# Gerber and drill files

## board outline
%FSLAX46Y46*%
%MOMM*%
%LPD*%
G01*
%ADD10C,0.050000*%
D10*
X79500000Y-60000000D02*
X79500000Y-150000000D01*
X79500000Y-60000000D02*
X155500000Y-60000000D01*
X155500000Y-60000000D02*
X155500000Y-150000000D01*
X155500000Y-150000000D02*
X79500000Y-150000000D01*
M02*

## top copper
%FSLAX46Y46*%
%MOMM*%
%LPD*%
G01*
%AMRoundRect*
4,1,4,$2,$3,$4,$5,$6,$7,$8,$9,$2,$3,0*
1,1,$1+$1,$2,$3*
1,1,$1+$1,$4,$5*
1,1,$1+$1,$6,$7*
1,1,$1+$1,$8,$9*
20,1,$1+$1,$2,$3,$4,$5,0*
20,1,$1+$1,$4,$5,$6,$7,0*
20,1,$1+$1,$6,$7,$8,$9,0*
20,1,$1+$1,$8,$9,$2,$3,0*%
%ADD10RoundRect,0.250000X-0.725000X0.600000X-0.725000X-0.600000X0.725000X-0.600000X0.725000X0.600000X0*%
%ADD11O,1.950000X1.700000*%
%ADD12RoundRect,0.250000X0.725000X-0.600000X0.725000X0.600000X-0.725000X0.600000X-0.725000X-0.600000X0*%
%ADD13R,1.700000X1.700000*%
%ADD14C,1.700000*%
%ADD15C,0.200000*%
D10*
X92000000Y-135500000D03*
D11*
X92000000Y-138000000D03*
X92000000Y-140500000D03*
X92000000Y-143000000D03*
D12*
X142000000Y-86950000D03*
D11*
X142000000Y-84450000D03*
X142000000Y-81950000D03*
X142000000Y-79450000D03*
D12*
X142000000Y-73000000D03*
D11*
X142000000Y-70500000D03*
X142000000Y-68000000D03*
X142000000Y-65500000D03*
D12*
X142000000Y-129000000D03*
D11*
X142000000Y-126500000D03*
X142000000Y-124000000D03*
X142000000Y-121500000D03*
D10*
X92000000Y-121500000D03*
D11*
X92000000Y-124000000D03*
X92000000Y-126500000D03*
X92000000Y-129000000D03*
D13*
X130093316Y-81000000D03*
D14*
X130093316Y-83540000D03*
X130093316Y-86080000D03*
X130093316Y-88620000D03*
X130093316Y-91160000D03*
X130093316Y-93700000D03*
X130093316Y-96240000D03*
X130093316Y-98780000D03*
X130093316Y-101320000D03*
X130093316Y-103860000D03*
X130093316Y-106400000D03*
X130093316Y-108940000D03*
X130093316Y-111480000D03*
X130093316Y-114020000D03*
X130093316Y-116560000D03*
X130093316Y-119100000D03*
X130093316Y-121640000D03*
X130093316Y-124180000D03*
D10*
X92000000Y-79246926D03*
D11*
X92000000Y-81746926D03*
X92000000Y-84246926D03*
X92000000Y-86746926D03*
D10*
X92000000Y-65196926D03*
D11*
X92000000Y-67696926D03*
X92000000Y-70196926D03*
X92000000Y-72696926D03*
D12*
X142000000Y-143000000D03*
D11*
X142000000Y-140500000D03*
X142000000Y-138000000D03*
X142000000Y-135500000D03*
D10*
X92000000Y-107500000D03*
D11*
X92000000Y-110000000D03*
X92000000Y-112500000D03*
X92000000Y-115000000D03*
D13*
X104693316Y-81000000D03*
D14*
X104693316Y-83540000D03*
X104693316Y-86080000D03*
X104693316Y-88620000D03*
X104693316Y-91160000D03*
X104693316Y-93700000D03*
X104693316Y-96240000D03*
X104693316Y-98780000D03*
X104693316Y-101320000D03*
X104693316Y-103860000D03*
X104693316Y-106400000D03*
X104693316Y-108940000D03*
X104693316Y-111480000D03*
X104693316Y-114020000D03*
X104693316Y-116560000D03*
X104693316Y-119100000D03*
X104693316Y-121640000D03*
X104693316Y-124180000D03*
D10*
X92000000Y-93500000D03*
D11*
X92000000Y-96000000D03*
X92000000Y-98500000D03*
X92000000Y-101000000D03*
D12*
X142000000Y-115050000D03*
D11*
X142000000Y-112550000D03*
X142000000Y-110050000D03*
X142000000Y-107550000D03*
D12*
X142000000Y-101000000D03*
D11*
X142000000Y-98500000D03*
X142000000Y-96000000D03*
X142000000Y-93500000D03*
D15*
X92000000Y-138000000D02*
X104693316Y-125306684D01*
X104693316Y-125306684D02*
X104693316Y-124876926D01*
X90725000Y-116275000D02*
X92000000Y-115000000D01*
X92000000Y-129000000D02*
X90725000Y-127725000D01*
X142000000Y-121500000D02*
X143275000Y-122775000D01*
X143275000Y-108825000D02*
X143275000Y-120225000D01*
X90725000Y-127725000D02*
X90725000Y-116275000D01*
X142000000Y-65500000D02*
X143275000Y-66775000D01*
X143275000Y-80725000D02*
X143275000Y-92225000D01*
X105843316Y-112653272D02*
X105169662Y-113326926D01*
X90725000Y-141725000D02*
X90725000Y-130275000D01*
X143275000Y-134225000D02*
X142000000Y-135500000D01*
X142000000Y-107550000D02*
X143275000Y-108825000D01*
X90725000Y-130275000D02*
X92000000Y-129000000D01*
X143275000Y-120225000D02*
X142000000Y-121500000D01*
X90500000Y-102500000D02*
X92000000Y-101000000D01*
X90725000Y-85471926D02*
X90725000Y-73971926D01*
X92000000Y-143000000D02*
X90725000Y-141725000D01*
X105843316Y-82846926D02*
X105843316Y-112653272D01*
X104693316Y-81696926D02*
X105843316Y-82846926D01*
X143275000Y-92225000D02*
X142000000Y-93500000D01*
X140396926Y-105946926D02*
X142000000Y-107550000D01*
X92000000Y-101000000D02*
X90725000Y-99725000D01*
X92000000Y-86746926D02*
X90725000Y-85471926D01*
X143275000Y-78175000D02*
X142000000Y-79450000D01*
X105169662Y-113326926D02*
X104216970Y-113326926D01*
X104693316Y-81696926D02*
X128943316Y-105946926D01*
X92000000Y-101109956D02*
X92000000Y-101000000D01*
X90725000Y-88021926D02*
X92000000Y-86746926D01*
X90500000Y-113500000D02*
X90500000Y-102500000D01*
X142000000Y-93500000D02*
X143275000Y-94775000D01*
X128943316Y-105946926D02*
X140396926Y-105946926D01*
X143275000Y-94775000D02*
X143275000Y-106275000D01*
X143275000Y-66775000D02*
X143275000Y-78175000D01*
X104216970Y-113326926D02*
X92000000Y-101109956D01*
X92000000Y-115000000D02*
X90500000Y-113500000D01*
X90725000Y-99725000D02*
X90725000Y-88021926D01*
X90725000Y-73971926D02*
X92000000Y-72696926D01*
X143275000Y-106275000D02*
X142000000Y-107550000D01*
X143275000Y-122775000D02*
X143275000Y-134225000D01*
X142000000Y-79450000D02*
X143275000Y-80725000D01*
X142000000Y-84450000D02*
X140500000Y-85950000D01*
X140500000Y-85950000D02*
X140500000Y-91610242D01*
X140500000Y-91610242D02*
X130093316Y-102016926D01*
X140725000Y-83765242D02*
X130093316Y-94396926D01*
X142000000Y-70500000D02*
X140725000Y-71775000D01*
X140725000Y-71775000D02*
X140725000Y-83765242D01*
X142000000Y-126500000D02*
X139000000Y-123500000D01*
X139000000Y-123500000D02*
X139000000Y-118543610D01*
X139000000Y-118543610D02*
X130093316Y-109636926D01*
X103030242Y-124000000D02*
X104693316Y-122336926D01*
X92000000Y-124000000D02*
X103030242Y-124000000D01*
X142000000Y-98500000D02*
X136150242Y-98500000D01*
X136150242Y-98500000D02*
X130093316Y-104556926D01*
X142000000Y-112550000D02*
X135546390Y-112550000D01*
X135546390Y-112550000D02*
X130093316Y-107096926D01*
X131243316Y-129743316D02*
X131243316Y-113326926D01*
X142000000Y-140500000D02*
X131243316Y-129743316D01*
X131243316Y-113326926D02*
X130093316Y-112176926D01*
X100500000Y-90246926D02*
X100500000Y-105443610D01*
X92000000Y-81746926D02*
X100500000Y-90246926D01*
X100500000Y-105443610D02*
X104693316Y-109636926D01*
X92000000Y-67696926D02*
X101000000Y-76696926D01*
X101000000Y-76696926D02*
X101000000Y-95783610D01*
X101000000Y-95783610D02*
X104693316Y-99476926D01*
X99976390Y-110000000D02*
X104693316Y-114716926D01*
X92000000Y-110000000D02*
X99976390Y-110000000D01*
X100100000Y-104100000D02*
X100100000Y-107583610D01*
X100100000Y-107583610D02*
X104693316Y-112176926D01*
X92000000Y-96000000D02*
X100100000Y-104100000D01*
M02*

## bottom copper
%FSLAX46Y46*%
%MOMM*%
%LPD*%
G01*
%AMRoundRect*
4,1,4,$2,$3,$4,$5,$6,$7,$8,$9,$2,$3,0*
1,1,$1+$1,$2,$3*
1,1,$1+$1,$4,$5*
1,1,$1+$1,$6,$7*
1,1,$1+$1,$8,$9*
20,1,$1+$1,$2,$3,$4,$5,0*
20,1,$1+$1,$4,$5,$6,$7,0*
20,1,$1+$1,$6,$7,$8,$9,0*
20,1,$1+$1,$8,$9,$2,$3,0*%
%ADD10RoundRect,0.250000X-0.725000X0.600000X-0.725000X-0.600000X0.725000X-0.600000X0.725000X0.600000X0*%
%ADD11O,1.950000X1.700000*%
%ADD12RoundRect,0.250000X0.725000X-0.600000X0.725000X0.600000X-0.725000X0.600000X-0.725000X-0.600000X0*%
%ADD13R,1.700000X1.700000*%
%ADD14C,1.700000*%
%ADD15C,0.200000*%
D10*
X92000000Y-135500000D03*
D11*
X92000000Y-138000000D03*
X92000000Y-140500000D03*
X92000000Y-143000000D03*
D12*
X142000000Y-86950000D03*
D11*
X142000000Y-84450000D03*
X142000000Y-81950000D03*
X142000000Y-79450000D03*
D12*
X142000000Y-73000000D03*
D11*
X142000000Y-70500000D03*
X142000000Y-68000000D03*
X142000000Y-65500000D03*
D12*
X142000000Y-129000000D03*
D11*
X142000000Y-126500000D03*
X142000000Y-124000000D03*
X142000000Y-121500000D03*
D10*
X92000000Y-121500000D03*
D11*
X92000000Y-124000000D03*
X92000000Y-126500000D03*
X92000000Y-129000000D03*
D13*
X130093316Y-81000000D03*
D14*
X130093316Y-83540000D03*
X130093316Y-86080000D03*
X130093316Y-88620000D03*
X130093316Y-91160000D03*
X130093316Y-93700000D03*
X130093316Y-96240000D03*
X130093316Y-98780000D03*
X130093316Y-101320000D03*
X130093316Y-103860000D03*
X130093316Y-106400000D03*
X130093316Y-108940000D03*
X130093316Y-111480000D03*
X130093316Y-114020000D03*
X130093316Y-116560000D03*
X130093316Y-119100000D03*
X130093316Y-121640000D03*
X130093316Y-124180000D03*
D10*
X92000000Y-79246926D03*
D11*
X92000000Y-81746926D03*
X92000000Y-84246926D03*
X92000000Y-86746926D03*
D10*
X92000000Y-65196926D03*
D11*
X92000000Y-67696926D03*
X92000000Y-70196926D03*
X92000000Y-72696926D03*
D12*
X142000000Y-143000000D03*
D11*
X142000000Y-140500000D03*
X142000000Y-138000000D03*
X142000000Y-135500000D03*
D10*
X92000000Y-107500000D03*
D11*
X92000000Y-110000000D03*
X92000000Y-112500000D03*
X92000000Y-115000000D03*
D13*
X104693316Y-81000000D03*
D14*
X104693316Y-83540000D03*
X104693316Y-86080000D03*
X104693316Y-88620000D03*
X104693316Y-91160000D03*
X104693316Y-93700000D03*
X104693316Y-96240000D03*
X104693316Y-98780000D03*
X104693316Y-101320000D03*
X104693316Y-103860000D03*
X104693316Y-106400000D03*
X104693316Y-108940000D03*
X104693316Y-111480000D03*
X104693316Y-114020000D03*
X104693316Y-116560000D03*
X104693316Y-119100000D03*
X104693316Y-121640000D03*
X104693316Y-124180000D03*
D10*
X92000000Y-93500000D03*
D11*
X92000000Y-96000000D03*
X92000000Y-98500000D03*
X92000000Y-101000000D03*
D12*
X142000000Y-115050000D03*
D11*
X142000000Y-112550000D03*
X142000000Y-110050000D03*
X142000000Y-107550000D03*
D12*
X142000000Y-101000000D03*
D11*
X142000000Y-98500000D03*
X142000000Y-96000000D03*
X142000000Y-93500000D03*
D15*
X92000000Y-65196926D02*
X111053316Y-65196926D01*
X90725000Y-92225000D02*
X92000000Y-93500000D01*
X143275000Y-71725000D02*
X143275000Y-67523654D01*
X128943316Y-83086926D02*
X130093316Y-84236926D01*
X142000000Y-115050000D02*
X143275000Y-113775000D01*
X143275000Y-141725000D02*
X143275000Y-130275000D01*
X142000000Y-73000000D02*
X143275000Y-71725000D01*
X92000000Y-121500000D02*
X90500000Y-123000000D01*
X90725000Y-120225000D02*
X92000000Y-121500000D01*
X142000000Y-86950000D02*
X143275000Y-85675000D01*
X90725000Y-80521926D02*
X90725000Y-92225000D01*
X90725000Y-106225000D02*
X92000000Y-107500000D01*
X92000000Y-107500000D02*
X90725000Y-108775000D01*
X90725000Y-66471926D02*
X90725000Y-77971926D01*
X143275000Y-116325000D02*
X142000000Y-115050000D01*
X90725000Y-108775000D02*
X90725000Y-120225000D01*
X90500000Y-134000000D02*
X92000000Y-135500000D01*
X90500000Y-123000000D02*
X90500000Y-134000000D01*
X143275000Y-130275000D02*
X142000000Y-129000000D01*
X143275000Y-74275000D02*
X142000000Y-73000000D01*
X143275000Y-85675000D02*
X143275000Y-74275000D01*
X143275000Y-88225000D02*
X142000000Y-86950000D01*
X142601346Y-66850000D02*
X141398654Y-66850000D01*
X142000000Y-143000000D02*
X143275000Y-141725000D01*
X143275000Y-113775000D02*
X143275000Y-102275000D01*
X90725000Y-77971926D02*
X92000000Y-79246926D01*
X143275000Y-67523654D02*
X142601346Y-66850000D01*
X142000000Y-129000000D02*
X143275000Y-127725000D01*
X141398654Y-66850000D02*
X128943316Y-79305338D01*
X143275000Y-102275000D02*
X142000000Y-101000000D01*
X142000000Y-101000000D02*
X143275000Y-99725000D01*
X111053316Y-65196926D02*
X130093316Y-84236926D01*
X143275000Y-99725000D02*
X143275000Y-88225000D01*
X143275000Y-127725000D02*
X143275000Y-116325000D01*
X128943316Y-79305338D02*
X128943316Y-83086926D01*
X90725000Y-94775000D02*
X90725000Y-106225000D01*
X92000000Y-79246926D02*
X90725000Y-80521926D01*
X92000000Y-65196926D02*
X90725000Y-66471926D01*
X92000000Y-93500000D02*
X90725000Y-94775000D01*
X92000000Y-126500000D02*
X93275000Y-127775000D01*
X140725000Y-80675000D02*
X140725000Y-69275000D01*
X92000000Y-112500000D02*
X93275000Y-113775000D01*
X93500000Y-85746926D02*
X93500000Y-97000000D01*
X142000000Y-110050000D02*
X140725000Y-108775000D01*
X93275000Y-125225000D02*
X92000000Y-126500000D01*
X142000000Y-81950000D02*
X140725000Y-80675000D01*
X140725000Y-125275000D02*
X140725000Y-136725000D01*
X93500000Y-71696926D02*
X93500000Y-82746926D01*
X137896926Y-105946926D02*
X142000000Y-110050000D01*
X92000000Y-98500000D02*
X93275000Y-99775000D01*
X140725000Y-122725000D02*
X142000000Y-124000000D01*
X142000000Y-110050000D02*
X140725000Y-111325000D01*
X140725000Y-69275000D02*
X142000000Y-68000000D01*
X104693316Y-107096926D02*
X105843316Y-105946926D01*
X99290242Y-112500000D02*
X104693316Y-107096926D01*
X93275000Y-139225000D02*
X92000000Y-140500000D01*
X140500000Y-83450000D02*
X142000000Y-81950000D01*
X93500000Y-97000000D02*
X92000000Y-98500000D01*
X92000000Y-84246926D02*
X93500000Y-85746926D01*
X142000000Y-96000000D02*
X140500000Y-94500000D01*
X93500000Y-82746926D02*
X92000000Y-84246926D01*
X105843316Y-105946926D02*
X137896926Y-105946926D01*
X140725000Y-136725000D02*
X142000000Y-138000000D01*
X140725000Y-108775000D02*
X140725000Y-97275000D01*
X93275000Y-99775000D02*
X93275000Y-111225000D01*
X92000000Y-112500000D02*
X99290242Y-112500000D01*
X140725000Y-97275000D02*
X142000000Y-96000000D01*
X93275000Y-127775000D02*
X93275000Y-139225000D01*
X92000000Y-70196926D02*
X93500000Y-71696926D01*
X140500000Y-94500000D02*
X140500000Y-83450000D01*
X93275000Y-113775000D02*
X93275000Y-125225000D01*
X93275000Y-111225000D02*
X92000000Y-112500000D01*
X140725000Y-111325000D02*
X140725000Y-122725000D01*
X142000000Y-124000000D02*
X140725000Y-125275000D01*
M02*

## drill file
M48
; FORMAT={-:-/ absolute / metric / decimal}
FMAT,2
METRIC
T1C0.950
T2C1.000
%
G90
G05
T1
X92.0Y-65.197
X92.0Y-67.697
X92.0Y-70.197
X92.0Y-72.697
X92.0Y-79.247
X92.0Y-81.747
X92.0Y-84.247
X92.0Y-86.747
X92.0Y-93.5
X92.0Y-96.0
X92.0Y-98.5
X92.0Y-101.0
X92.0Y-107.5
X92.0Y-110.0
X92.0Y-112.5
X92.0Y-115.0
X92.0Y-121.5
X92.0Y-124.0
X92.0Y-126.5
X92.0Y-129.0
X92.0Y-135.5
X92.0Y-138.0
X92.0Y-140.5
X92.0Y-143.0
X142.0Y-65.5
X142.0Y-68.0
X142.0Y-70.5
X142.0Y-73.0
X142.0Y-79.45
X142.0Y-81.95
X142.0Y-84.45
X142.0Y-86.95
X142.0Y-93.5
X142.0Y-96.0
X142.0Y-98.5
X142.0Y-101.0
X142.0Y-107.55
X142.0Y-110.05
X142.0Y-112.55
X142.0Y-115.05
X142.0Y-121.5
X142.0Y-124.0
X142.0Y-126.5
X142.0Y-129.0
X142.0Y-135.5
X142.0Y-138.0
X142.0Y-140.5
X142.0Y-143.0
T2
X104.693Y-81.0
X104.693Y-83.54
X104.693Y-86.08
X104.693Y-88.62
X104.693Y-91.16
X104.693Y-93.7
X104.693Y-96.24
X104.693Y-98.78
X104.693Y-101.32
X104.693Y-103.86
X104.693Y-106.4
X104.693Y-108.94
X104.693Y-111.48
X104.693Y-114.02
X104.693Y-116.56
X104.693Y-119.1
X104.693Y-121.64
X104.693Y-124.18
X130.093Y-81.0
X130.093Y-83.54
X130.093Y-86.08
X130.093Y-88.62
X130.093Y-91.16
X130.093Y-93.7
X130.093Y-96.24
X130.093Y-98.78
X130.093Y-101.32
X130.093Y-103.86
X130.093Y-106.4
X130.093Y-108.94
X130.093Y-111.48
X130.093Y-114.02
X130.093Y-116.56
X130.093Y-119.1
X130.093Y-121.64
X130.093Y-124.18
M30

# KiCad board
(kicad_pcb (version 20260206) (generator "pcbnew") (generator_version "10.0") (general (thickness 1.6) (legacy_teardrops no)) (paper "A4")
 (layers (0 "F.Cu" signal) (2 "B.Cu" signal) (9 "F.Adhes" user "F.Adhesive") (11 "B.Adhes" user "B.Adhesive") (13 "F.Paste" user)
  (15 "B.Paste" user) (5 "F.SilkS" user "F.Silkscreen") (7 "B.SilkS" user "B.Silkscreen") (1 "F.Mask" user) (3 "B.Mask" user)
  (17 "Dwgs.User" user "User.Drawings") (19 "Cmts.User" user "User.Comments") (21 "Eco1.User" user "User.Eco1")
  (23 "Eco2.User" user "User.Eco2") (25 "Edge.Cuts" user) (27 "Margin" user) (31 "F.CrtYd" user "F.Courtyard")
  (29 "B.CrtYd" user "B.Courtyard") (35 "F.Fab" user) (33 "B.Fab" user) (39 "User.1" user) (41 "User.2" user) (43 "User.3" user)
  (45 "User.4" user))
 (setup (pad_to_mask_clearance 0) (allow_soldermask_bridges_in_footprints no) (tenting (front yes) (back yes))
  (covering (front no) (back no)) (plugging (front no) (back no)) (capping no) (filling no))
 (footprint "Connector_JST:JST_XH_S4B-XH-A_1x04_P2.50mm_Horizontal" (layer "F.Cu") (at 92 135.5 -90)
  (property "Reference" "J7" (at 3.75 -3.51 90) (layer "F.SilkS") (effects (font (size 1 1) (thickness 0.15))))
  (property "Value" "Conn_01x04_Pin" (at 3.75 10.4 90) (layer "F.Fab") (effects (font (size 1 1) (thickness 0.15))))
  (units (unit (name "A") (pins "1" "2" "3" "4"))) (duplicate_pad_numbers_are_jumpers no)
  (pad "1" thru_hole roundrect (at 0 0 270) (size 1.7 1.95) (drill 0.95) (layers "*.Cu" "*.Mask") (remove_unused_layers no)
   (roundrect_rratio 0.147059) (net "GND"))
  (pad "2" thru_hole oval (at 2.5 0 270) (size 1.7 1.95) (drill 0.95) (layers "*.Cu" "*.Mask") (remove_unused_layers no) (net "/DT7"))
  (pad "3" thru_hole oval (at 5 0 270) (size 1.7 1.95) (drill 0.95) (layers "*.Cu" "*.Mask") (remove_unused_layers no) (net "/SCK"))
  (pad "4" thru_hole oval (at 7.5 0 270) (size 1.7 1.95) (drill 0.95) (layers "*.Cu" "*.Mask") (remove_unused_layers no) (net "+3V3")))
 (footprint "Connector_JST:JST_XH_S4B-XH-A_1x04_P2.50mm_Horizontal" (layer "F.Cu") (at 142 86.95 90)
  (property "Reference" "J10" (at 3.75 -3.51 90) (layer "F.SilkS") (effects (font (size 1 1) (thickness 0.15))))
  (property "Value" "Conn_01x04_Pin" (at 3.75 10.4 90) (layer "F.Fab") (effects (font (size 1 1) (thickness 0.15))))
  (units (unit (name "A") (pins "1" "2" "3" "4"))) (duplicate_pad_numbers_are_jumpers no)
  (pad "1" thru_hole roundrect (at 0 0 90) (size 1.7 1.95) (drill 0.95) (layers "*.Cu" "*.Mask") (remove_unused_layers no)
   (roundrect_rratio 0.147059) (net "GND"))
  (pad "2" thru_hole oval (at 2.5 0 90) (size 1.7 1.95) (drill 0.95) (layers "*.Cu" "*.Mask") (remove_unused_layers no) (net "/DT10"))
  (pad "3" thru_hole oval (at 5 0 90) (size 1.7 1.95) (drill 0.95) (layers "*.Cu" "*.Mask") (remove_unused_layers no) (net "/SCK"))
  (pad "4" thru_hole oval (at 7.5 0 90) (size 1.7 1.95) (drill 0.95) (layers "*.Cu" "*.Mask") (remove_unused_layers no) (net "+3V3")))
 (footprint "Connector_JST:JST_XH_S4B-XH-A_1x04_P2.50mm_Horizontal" (layer "F.Cu") (at 142 73 90)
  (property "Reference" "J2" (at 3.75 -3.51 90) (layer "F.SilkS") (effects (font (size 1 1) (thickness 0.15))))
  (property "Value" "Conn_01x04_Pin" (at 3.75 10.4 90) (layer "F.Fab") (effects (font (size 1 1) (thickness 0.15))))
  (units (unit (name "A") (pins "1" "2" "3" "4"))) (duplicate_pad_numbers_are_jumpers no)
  (pad "1" thru_hole roundrect (at 0 0 90) (size 1.7 1.95) (drill 0.95) (layers "*.Cu" "*.Mask") (remove_unused_layers no)
   (roundrect_rratio 0.147059) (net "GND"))
  (pad "2" thru_hole oval (at 2.5 0 90) (size 1.7 1.95) (drill 0.95) (layers "*.Cu" "*.Mask") (remove_unused_layers no) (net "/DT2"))
  (pad "3" thru_hole oval (at 5 0 90) (size 1.7 1.95) (drill 0.95) (layers "*.Cu" "*.Mask") (remove_unused_layers no) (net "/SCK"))
  (pad "4" thru_hole oval (at 7.5 0 90) (size 1.7 1.95) (drill 0.95) (layers "*.Cu" "*.Mask") (remove_unused_layers no) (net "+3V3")))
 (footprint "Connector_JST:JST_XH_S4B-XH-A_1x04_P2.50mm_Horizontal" (layer "F.Cu") (at 142 129 90)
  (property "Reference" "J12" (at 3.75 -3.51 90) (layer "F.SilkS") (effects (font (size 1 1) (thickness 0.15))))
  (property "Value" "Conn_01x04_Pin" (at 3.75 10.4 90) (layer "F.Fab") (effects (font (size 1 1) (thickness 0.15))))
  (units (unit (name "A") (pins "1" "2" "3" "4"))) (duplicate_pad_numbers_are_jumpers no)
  (pad "1" thru_hole roundrect (at 0 0 90) (size 1.7 1.95) (drill 0.95) (layers "*.Cu" "*.Mask") (remove_unused_layers no)
   (roundrect_rratio 0.147059) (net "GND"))
  (pad "2" thru_hole oval (at 2.5 0 90) (size 1.7 1.95) (drill 0.95) (layers "*.Cu" "*.Mask") (remove_unused_layers no) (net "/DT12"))
  (pad "3" thru_hole oval (at 5 0 90) (size 1.7 1.95) (drill 0.95) (layers "*.Cu" "*.Mask") (remove_unused_layers no) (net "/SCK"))
  (pad "4" thru_hole oval (at 7.5 0 90) (size 1.7 1.95) (drill 0.95) (layers "*.Cu" "*.Mask") (remove_unused_layers no) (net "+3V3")))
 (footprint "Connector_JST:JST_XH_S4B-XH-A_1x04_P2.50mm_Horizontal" (layer "F.Cu") (at 92 121.5 -90)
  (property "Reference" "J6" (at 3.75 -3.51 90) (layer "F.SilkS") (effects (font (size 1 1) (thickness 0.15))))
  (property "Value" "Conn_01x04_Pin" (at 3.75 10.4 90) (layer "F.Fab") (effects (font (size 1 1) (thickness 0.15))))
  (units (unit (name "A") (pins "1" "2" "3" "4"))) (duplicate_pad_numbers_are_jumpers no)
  (pad "1" thru_hole roundrect (at 0 0 270) (size 1.7 1.95) (drill 0.95) (layers "*.Cu" "*.Mask") (remove_unused_layers no)
   (roundrect_rratio 0.147059) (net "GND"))
  (pad "2" thru_hole oval (at 2.5 0 270) (size 1.7 1.95) (drill 0.95) (layers "*.Cu" "*.Mask") (remove_unused_layers no) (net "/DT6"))
  (pad "3" thru_hole oval (at 5 0 270) (size 1.7 1.95) (drill 0.95) (layers "*.Cu" "*.Mask") (remove_unused_layers no) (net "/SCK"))
  (pad "4" thru_hole oval (at 7.5 0 270) (size 1.7 1.95) (drill 0.95) (layers "*.Cu" "*.Mask") (remove_unused_layers no) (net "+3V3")))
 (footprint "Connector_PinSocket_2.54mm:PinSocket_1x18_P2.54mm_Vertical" (layer "F.Cu") (at 130.093316 81)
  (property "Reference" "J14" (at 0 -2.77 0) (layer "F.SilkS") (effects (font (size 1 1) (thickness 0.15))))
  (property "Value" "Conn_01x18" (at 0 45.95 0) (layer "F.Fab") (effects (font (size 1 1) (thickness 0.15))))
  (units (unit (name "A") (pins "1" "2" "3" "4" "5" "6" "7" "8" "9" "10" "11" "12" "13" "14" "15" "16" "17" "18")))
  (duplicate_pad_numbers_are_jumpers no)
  (pad "1" thru_hole rect (at 0 0) (size 1.7 1.7) (drill 1) (layers "*.Cu" "*.Mask") (remove_unused_layers no)
   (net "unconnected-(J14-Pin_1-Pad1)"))
  (pad "2" thru_hole circle (at 0 2.54) (size 1.7 1.7) (drill 1) (layers "*.Cu" "*.Mask") (remove_unused_layers no) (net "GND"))
  (pad "3" thru_hole circle (at 0 5.08) (size 1.7 1.7) (drill 1) (layers "*.Cu" "*.Mask") (remove_unused_layers no)
   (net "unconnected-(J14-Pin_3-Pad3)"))
  (pad "4" thru_hole circle (at 0 7.62) (size 1.7 1.7) (drill 1) (layers "*.Cu" "*.Mask") (remove_unused_layers no)
   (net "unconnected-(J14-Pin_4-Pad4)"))
  (pad "5" thru_hole circle (at 0 10.16) (size 1.7 1.7) (drill 1) (layers "*.Cu" "*.Mask") (remove_unused_layers no)
   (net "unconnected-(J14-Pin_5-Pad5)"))
  (pad "6" thru_hole circle (at 0 12.7) (size 1.7 1.7) (drill 1) (layers "*.Cu" "*.Mask") (remove_unused_layers no) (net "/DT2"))
  (pad "7" thru_hole circle (at 0 15.24) (size 1.7 1.7) (drill 1) (layers "*.Cu" "*.Mask") (remove_unused_layers no)
   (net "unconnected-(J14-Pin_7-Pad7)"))
  (pad "8" thru_hole circle (at 0 17.78) (size 1.7 1.7) (drill 1) (layers "*.Cu" "*.Mask") (remove_unused_layers no)
   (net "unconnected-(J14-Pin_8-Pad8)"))
  (pad "9" thru_hole circle (at 0 20.32) (size 1.7 1.7) (drill 1) (layers "*.Cu" "*.Mask") (remove_unused_layers no) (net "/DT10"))
  (pad "10" thru_hole circle (at 0 22.86) (size 1.7 1.7) (drill 1) (layers "*.Cu" "*.Mask") (remove_unused_layers no) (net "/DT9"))
  (pad "11" thru_hole circle (at 0 25.4) (size 1.7 1.7) (drill 1) (layers "*.Cu" "*.Mask") (remove_unused_layers no) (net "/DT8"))
  (pad "12" thru_hole circle (at 0 27.94) (size 1.7 1.7) (drill 1) (layers "*.Cu" "*.Mask") (remove_unused_layers no) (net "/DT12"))
  (pad "13" thru_hole circle (at 0 30.48) (size 1.7 1.7) (drill 1) (layers "*.Cu" "*.Mask") (remove_unused_layers no) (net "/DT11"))
  (pad "14" thru_hole circle (at 0 33.02) (size 1.7 1.7) (drill 1) (layers "*.Cu" "*.Mask") (remove_unused_layers no)
   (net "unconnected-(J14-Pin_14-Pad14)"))
  (pad "15" thru_hole circle (at 0 35.56) (size 1.7 1.7) (drill 1) (layers "*.Cu" "*.Mask") (remove_unused_layers no)
   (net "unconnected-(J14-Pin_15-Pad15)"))
  (pad "16" thru_hole circle (at 0 38.1) (size 1.7 1.7) (drill 1) (layers "*.Cu" "*.Mask") (remove_unused_layers no)
   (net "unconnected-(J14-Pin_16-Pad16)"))
  (pad "17" thru_hole circle (at 0 40.64) (size 1.7 1.7) (drill 1) (layers "*.Cu" "*.Mask") (remove_unused_layers no)
   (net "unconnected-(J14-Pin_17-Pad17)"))
  (pad "18" thru_hole circle (at 0 43.18) (size 1.7 1.7) (drill 1) (layers "*.Cu" "*.Mask") (remove_unused_layers no)
   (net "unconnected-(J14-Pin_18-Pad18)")))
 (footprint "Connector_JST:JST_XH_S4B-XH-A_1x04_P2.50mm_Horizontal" (layer "F.Cu") (at 92 79.246926 -90)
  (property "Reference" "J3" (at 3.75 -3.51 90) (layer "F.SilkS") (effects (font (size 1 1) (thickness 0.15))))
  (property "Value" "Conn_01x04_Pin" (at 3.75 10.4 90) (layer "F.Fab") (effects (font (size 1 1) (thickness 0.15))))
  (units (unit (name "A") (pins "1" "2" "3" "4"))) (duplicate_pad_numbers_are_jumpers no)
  (pad "1" thru_hole roundrect (at 0 0 270) (size 1.7 1.95) (drill 0.95) (layers "*.Cu" "*.Mask") (remove_unused_layers no)
   (roundrect_rratio 0.147059) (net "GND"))
  (pad "2" thru_hole oval (at 2.5 0 270) (size 1.7 1.95) (drill 0.95) (layers "*.Cu" "*.Mask") (remove_unused_layers no) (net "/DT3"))
  (pad "3" thru_hole oval (at 5 0 270) (size 1.7 1.95) (drill 0.95) (layers "*.Cu" "*.Mask") (remove_unused_layers no) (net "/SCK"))
  (pad "4" thru_hole oval (at 7.5 0 270) (size 1.7 1.95) (drill 0.95) (layers "*.Cu" "*.Mask") (remove_unused_layers no) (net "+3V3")))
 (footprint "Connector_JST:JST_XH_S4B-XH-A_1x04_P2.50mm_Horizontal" (layer "F.Cu") (at 92 65.196926 -90)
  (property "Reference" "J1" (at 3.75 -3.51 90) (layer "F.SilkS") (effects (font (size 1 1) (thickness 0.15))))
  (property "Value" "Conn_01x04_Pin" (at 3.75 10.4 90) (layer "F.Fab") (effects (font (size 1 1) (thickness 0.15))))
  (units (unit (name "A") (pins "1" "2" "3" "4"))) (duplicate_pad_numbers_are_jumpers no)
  (pad "1" thru_hole roundrect (at 0 0 270) (size 1.7 1.95) (drill 0.95) (layers "*.Cu" "*.Mask") (remove_unused_layers no)
   (roundrect_rratio 0.147059) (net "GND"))
  (pad "2" thru_hole oval (at 2.5 0 270) (size 1.7 1.95) (drill 0.95) (layers "*.Cu" "*.Mask") (remove_unused_layers no) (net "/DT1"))
  (pad "3" thru_hole oval (at 5 0 270) (size 1.7 1.95) (drill 0.95) (layers "*.Cu" "*.Mask") (remove_unused_layers no) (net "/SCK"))
  (pad "4" thru_hole oval (at 7.5 0 270) (size 1.7 1.95) (drill 0.95) (layers "*.Cu" "*.Mask") (remove_unused_layers no) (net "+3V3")))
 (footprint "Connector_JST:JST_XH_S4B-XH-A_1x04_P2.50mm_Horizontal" (layer "F.Cu") (at 142 143 90)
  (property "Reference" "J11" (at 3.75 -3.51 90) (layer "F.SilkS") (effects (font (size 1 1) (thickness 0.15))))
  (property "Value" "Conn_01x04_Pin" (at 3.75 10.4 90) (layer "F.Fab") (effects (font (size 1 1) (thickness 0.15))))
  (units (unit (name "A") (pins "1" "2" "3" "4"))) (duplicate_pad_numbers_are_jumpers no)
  (pad "1" thru_hole roundrect (at 0 0 90) (size 1.7 1.95) (drill 0.95) (layers "*.Cu" "*.Mask") (remove_unused_layers no)
   (roundrect_rratio 0.147059) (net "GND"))
  (pad "2" thru_hole oval (at 2.5 0 90) (size 1.7 1.95) (drill 0.95) (layers "*.Cu" "*.Mask") (remove_unused_layers no) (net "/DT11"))
  (pad "3" thru_hole oval (at 5 0 90) (size 1.7 1.95) (drill 0.95) (layers "*.Cu" "*.Mask") (remove_unused_layers no) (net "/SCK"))
  (pad "4" thru_hole oval (at 7.5 0 90) (size 1.7 1.95) (drill 0.95) (layers "*.Cu" "*.Mask") (remove_unused_layers no) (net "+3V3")))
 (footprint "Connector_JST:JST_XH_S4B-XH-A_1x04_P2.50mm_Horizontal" (layer "F.Cu") (at 92 107.5 -90)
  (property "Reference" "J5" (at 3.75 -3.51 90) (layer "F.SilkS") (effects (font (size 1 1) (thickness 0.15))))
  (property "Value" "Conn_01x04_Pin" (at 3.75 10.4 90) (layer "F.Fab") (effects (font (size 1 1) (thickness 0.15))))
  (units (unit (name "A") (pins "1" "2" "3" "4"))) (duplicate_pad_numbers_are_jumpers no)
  (pad "1" thru_hole roundrect (at 0 0 270) (size 1.7 1.95) (drill 0.95) (layers "*.Cu" "*.Mask") (remove_unused_layers no)
   (roundrect_rratio 0.147059) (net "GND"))
  (pad "2" thru_hole oval (at 2.5 0 270) (size 1.7 1.95) (drill 0.95) (layers "*.Cu" "*.Mask") (remove_unused_layers no) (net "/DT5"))
  (pad "3" thru_hole oval (at 5 0 270) (size 1.7 1.95) (drill 0.95) (layers "*.Cu" "*.Mask") (remove_unused_layers no) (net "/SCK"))
  (pad "4" thru_hole oval (at 7.5 0 270) (size 1.7 1.95) (drill 0.95) (layers "*.Cu" "*.Mask") (remove_unused_layers no) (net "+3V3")))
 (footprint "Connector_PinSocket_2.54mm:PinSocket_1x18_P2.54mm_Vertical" (layer "F.Cu") (at 104.693316 81)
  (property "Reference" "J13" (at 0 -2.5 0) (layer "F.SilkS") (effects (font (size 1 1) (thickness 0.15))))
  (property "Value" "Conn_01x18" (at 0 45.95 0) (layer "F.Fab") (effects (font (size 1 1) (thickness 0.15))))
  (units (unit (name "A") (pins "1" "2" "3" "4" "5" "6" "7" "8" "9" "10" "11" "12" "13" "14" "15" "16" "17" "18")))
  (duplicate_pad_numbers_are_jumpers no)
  (pad "1" thru_hole rect (at 0 0) (size 1.7 1.7) (drill 1) (layers "*.Cu" "*.Mask") (remove_unused_layers no) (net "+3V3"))
  (pad "2" thru_hole circle (at 0 2.54) (size 1.7 1.7) (drill 1) (layers "*.Cu" "*.Mask") (remove_unused_layers no)
   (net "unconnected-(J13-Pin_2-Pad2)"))
  (pad "3" thru_hole circle (at 0 5.08) (size 1.7 1.7) (drill 1) (layers "*.Cu" "*.Mask") (remove_unused_layers no)
   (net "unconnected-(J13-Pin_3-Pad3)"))
  (pad "4" thru_hole circle (at 0 7.62) (size 1.7 1.7) (drill 1) (layers "*.Cu" "*.Mask") (remove_unused_layers no)
   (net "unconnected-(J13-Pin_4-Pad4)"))
  (pad "5" thru_hole circle (at 0 10.16) (size 1.7 1.7) (drill 1) (layers "*.Cu" "*.Mask") (remove_unused_layers no)
   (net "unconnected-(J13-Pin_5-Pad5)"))
  (pad "6" thru_hole circle (at 0 12.7) (size 1.7 1.7) (drill 1) (layers "*.Cu" "*.Mask") (remove_unused_layers no)
   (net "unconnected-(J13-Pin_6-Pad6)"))
  (pad "7" thru_hole circle (at 0 15.24) (size 1.7 1.7) (drill 1) (layers "*.Cu" "*.Mask") (remove_unused_layers no)
   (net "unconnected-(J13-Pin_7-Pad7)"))
  (pad "8" thru_hole circle (at 0 17.78) (size 1.7 1.7) (drill 1) (layers "*.Cu" "*.Mask") (remove_unused_layers no) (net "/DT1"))
  (pad "9" thru_hole circle (at 0 20.32) (size 1.7 1.7) (drill 1) (layers "*.Cu" "*.Mask") (remove_unused_layers no)
   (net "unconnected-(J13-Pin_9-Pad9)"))
  (pad "10" thru_hole circle (at 0 22.86) (size 1.7 1.7) (drill 1) (layers "*.Cu" "*.Mask") (remove_unused_layers no)
   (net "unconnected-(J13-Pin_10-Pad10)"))
  (pad "11" thru_hole circle (at 0 25.4) (size 1.7 1.7) (drill 1) (layers "*.Cu" "*.Mask") (remove_unused_layers no) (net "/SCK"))
  (pad "12" thru_hole circle (at 0 27.94) (size 1.7 1.7) (drill 1) (layers "*.Cu" "*.Mask") (remove_unused_layers no) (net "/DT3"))
  (pad "13" thru_hole circle (at 0 30.48) (size 1.7 1.7) (drill 1) (layers "*.Cu" "*.Mask") (remove_unused_layers no) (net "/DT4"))
  (pad "14" thru_hole circle (at 0 33.02) (size 1.7 1.7) (drill 1) (layers "*.Cu" "*.Mask") (remove_unused_layers no) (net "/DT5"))
  (pad "15" thru_hole circle (at 0 35.56) (size 1.7 1.7) (drill 1) (layers "*.Cu" "*.Mask") (remove_unused_layers no)
   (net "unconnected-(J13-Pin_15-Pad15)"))
  (pad "16" thru_hole circle (at 0 38.1) (size 1.7 1.7) (drill 1) (layers "*.Cu" "*.Mask") (remove_unused_layers no)
   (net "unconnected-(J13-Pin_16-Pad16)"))
  (pad "17" thru_hole circle (at 0 40.64) (size 1.7 1.7) (drill 1) (layers "*.Cu" "*.Mask") (remove_unused_layers no) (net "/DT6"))
  (pad "18" thru_hole circle (at 0 43.18) (size 1.7 1.7) (drill 1) (layers "*.Cu" "*.Mask") (remove_unused_layers no) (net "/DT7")))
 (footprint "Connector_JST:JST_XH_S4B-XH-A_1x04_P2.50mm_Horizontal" (layer "F.Cu") (at 92 93.5 -90)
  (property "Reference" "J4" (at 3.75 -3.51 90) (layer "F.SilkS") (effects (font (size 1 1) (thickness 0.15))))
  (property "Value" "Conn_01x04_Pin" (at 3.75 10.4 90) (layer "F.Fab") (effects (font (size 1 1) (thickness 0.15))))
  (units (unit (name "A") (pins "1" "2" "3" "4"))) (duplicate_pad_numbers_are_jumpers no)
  (pad "1" thru_hole roundrect (at 0 0 270) (size 1.7 1.95) (drill 0.95) (layers "*.Cu" "*.Mask") (remove_unused_layers no)
   (roundrect_rratio 0.147059) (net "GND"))
  (pad "2" thru_hole oval (at 2.5 0 270) (size 1.7 1.95) (drill 0.95) (layers "*.Cu" "*.Mask") (remove_unused_layers no) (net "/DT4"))
  (pad "3" thru_hole oval (at 5 0 270) (size 1.7 1.95) (drill 0.95) (layers "*.Cu" "*.Mask") (remove_unused_layers no) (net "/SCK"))
  (pad "4" thru_hole oval (at 7.5 0 270) (size 1.7 1.95) (drill 0.95) (layers "*.Cu" "*.Mask") (remove_unused_layers no) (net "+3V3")))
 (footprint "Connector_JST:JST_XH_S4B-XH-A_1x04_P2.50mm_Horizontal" (layer "F.Cu") (at 142 115.05 90)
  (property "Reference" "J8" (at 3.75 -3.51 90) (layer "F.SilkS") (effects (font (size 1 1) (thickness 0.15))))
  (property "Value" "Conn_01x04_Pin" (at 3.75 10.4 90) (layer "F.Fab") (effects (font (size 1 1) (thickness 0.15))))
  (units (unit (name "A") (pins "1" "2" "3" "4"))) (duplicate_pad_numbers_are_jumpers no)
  (pad "1" thru_hole roundrect (at 0 0 90) (size 1.7 1.95) (drill 0.95) (layers "*.Cu" "*.Mask") (remove_unused_layers no)
   (roundrect_rratio 0.147059) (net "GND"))
  (pad "2" thru_hole oval (at 2.5 0 90) (size 1.7 1.95) (drill 0.95) (layers "*.Cu" "*.Mask") (remove_unused_layers no) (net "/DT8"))
  (pad "3" thru_hole oval (at 5 0 90) (size 1.7 1.95) (drill 0.95) (layers "*.Cu" "*.Mask") (remove_unused_layers no) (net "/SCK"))
  (pad "4" thru_hole oval (at 7.5 0 90) (size 1.7 1.95) (drill 0.95) (layers "*.Cu" "*.Mask") (remove_unused_layers no) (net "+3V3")))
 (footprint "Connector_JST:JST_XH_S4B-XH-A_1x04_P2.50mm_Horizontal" (layer "F.Cu") (at 142 101 90)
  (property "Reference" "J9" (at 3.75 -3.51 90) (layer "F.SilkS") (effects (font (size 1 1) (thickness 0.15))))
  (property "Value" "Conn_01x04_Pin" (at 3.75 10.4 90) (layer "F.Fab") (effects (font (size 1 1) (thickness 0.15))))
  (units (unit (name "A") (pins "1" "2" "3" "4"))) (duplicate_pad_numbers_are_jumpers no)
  (pad "1" thru_hole roundrect (at 0 0 90) (size 1.7 1.95) (drill 0.95) (layers "*.Cu" "*.Mask") (remove_unused_layers no)
   (roundrect_rratio 0.147059) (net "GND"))
  (pad "2" thru_hole oval (at 2.5 0 90) (size 1.7 1.95) (drill 0.95) (layers "*.Cu" "*.Mask") (remove_unused_layers no) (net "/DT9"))
  (pad "3" thru_hole oval (at 5 0 90) (size 1.7 1.95) (drill 0.95) (layers "*.Cu" "*.Mask") (remove_unused_layers no) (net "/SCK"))
  (pad "4" thru_hole oval (at 7.5 0 90) (size 1.7 1.95) (drill 0.95) (layers "*.Cu" "*.Mask") (remove_unused_layers no) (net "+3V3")))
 (gr_line (start 79.5 60) (end 79.5 150) (stroke (width 0.05) (type default)) (layer "Edge.Cuts"))
 (gr_line (start 79.5 60) (end 155.5 60) (stroke (width 0.05) (type default)) (layer "Edge.Cuts"))
 (gr_line (start 155.5 60) (end 155.5 150) (stroke (width 0.05) (type default)) (layer "Edge.Cuts"))
 (gr_line (start 155.5 150) (end 79.5 150) (stroke (width 0.05) (type default)) (layer "Edge.Cuts"))
 (segment (start 92 65.196926) (end 111.053316 65.196926) (width 0.2) (layer "B.Cu") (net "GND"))
 (segment (start 90.725 92.225) (end 92 93.5) (width 0.2) (layer "B.Cu") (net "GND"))
 (segment (start 143.275 71.725) (end 143.275 67.523654) (width 0.2) (layer "B.Cu") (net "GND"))
 (segment (start 128.943316 83.086926) (end 130.093316 84.236926) (width 0.2) (layer "B.Cu") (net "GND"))
 (segment (start 142 115.05) (end 143.275 113.775) (width 0.2) (layer "B.Cu") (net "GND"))
 (segment (start 143.275 141.725) (end 143.275 130.275) (width 0.2) (layer "B.Cu") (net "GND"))
 (segment (start 142 73) (end 143.275 71.725) (width 0.2) (layer "B.Cu") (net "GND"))
 (segment (start 92 121.5) (end 90.5 123) (width 0.2) (layer "B.Cu") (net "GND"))
 (segment (start 90.725 120.225) (end 92 121.5) (width 0.2) (layer "B.Cu") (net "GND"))
 (segment (start 142 86.95) (end 143.275 85.675) (width 0.2) (layer "B.Cu") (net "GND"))
 (segment (start 90.725 80.521926) (end 90.725 92.225) (width 0.2) (layer "B.Cu") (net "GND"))
 (segment (start 90.725 106.225) (end 92 107.5) (width 0.2) (layer "B.Cu") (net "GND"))
 (segment (start 92 107.5) (end 90.725 108.775) (width 0.2) (layer "B.Cu") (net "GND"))
 (segment (start 90.725 66.471926) (end 90.725 77.971926) (width 0.2) (layer "B.Cu") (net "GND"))
 (segment (start 143.275 116.325) (end 142 115.05) (width 0.2) (layer "B.Cu") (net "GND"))
 (segment (start 90.725 108.775) (end 90.725 120.225) (width 0.2) (layer "B.Cu") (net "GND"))
 (segment (start 90.5 134) (end 92 135.5) (width 0.2) (layer "B.Cu") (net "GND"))
 (segment (start 90.5 123) (end 90.5 134) (width 0.2) (layer "B.Cu") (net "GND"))
 (segment (start 143.275 130.275) (end 142 129) (width 0.2) (layer "B.Cu") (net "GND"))
 (segment (start 143.275 74.275) (end 142 73) (width 0.2) (layer "B.Cu") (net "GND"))
 (segment (start 143.275 85.675) (end 143.275 74.275) (width 0.2) (layer "B.Cu") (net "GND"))
 (segment (start 143.275 88.225) (end 142 86.95) (width 0.2) (layer "B.Cu") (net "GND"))
 (segment (start 142.601346 66.85) (end 141.398654 66.85) (width 0.2) (layer "B.Cu") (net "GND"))
 (segment (start 142 143) (end 143.275 141.725) (width 0.2) (layer "B.Cu") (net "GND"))
 (segment (start 143.275 113.775) (end 143.275 102.275) (width 0.2) (layer "B.Cu") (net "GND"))
 (segment (start 90.725 77.971926) (end 92 79.246926) (width 0.2) (layer "B.Cu") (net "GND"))
 (segment (start 143.275 67.523654) (end 142.601346 66.85) (width 0.2) (layer "B.Cu") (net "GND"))
 (segment (start 142 129) (end 143.275 127.725) (width 0.2) (layer "B.Cu") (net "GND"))
 (segment (start 141.398654 66.85) (end 128.943316 79.305338) (width 0.2) (layer "B.Cu") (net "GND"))
 (segment (start 143.275 102.275) (end 142 101) (width 0.2) (layer "B.Cu") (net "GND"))
 (segment (start 142 101) (end 143.275 99.725) (width 0.2) (layer "B.Cu") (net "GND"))
 (segment (start 111.053316 65.196926) (end 130.093316 84.236926) (width 0.2) (layer "B.Cu") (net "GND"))
 (segment (start 143.275 99.725) (end 143.275 88.225) (width 0.2) (layer "B.Cu") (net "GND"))
 (segment (start 143.275 127.725) (end 143.275 116.325) (width 0.2) (layer "B.Cu") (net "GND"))
 (segment (start 128.943316 79.305338) (end 128.943316 83.086926) (width 0.2) (layer "B.Cu") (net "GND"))
 (segment (start 90.725 94.775) (end 90.725 106.225) (width 0.2) (layer "B.Cu") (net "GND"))
 (segment (start 92 79.246926) (end 90.725 80.521926) (width 0.2) (layer "B.Cu") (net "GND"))
 (segment (start 92 65.196926) (end 90.725 66.471926) (width 0.2) (layer "B.Cu") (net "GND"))
 (segment (start 92 93.5) (end 90.725 94.775) (width 0.2) (layer "B.Cu") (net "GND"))
 (segment (start 92 138) (end 104.693316 125.306684) (width 0.2) (layer "F.Cu") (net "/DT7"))
 (segment (start 104.693316 125.306684) (end 104.693316 124.876926) (width 0.2) (layer "F.Cu") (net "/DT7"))
 (segment (start 92 126.5) (end 93.275 127.775) (width 0.2) (layer "B.Cu") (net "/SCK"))
 (segment (start 140.725 80.675) (end 140.725 69.275) (width 0.2) (layer "B.Cu") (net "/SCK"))
 (segment (start 92 112.5) (end 93.275 113.775) (width 0.2) (layer "B.Cu") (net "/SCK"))
 (segment (start 93.5 85.746926) (end 93.5 97) (width 0.2) (layer "B.Cu") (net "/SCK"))
 (segment (start 142 110.05) (end 140.725 108.775) (width 0.2) (layer "B.Cu") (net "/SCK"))
 (segment (start 93.275 125.225) (end 92 126.5) (width 0.2) (layer "B.Cu") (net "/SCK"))
 (segment (start 142 81.95) (end 140.725 80.675) (width 0.2) (layer "B.Cu") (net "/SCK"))
 (segment (start 140.725 125.275) (end 140.725 136.725) (width 0.2) (layer "B.Cu") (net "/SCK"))
 (segment (start 93.5 71.696926) (end 93.5 82.746926) (width 0.2) (layer "B.Cu") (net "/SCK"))
 (segment (start 137.896926 105.946926) (end 142 110.05) (width 0.2) (layer "B.Cu") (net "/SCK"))
 (segment (start 92 98.5) (end 93.275 99.775) (width 0.2) (layer "B.Cu") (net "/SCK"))
 (segment (start 140.725 122.725) (end 142 124) (width 0.2) (layer "B.Cu") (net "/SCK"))
 (segment (start 142 110.05) (end 140.725 111.325) (width 0.2) (layer "B.Cu") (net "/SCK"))
 (segment (start 140.725 69.275) (end 142 68) (width 0.2) (layer "B.Cu") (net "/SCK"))
 (segment (start 104.693316 107.096926) (end 105.843316 105.946926) (width 0.2) (layer "B.Cu") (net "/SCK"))
 (segment (start 99.290242 112.5) (end 104.693316 107.096926) (width 0.2) (layer "B.Cu") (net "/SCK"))
 (segment (start 93.275 139.225) (end 92 140.5) (width 0.2) (layer "B.Cu") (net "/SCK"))
 (segment (start 140.5 83.45) (end 142 81.95) (width 0.2) (layer "B.Cu") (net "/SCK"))
 (segment (start 93.5 97) (end 92 98.5) (width 0.2) (layer "B.Cu") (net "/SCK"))
 (segment (start 92 84.246926) (end 93.5 85.746926) (width 0.2) (layer "B.Cu") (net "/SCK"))
 (segment (start 142 96) (end 140.5 94.5) (width 0.2) (layer "B.Cu") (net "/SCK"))
 (segment (start 93.5 82.746926) (end 92 84.246926) (width 0.2) (layer "B.Cu") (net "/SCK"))
 (segment (start 105.843316 105.946926) (end 137.896926 105.946926) (width 0.2) (layer "B.Cu") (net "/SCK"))
 (segment (start 140.725 136.725) (end 142 138) (width 0.2) (layer "B.Cu") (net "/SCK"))
 (segment (start 140.725 108.775) (end 140.725 97.275) (width 0.2) (layer "B.Cu") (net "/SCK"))
 (segment (start 93.275 99.775) (end 93.275 111.225) (width 0.2) (layer "B.Cu") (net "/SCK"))
 (segment (start 92 112.5) (end 99.290242 112.5) (width 0.2) (layer "B.Cu") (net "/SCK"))
 (segment (start 140.725 97.275) (end 142 96) (width 0.2) (layer "B.Cu") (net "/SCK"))
 (segment (start 93.275 127.775) (end 93.275 139.225) (width 0.2) (layer "B.Cu") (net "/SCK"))
 (segment (start 92 70.196926) (end 93.5 71.696926) (width 0.2) (layer "B.Cu") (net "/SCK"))
 (segment (start 140.5 94.5) (end 140.5 83.45) (width 0.2) (layer "B.Cu") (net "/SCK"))
 (segment (start 93.275 113.775) (end 93.275 125.225) (width 0.2) (layer "B.Cu") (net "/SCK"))
 (segment (start 93.275 111.225) (end 92 112.5) (width 0.2) (layer "B.Cu") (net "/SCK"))
 (segment (start 140.725 111.325) (end 140.725 122.725) (width 0.2) (layer "B.Cu") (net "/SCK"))
 (segment (start 142 124) (end 140.725 125.275) (width 0.2) (layer "B.Cu") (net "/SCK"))
 (segment (start 90.725 116.275) (end 92 115) (width 0.2) (layer "F.Cu") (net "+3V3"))
 (segment (start 92 129) (end 90.725 127.725) (width 0.2) (layer "F.Cu") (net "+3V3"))
 (segment (start 142 121.5) (end 143.275 122.775) (width 0.2) (layer "F.Cu") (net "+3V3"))
 (segment (start 143.275 108.825) (end 143.275 120.225) (width 0.2) (layer "F.Cu") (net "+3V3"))
 (segment (start 90.725 127.725) (end 90.725 116.275) (width 0.2) (layer "F.Cu") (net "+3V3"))
 (segment (start 142 65.5) (end 143.275 66.775) (width 0.2) (layer "F.Cu") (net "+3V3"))
 (segment (start 143.275 80.725) (end 143.275 92.225) (width 0.2) (layer "F.Cu") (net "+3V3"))
 (segment (start 105.843316 112.653272) (end 105.169662 113.326926) (width 0.2) (layer "F.Cu") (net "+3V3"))
 (segment (start 90.725 141.725) (end 90.725 130.275) (width 0.2) (layer "F.Cu") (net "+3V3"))
 (segment (start 143.275 134.225) (end 142 135.5) (width 0.2) (layer "F.Cu") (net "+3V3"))
 (segment (start 142 107.55) (end 143.275 108.825) (width 0.2) (layer "F.Cu") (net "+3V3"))
 (segment (start 90.725 130.275) (end 92 129) (width 0.2) (layer "F.Cu") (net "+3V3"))
 (segment (start 143.275 120.225) (end 142 121.5) (width 0.2) (layer "F.Cu") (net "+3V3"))
 (segment (start 90.5 102.5) (end 92 101) (width 0.2) (layer "F.Cu") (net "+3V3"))
 (segment (start 90.725 85.471926) (end 90.725 73.971926) (width 0.2) (layer "F.Cu") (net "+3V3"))
 (segment (start 92 143) (end 90.725 141.725) (width 0.2) (layer "F.Cu") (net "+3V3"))
 (segment (start 105.843316 82.846926) (end 105.843316 112.653272) (width 0.2) (layer "F.Cu") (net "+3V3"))
 (segment (start 104.693316 81.696926) (end 105.843316 82.846926) (width 0.2) (layer "F.Cu") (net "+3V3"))
 (segment (start 143.275 92.225) (end 142 93.5) (width 0.2) (layer "F.Cu") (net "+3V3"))
 (segment (start 140.396926 105.946926) (end 142 107.55) (width 0.2) (layer "F.Cu") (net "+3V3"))
 (segment (start 92 101) (end 90.725 99.725) (width 0.2) (layer "F.Cu") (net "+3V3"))
 (segment (start 92 86.746926) (end 90.725 85.471926) (width 0.2) (layer "F.Cu") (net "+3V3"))
 (segment (start 143.275 78.175) (end 142 79.45) (width 0.2) (layer "F.Cu") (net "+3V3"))
 (segment (start 105.169662 113.326926) (end 104.21697 113.326926) (width 0.2) (layer "F.Cu") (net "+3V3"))
 (segment (start 104.693316 81.696926) (end 128.943316 105.946926) (width 0.2) (layer "F.Cu") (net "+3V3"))
 (segment (start 92 101.109956) (end 92 101) (width 0.2) (layer "F.Cu") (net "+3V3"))
 (segment (start 90.725 88.021926) (end 92 86.746926) (width 0.2) (layer "F.Cu") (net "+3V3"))
 (segment (start 90.5 113.5) (end 90.5 102.5) (width 0.2) (layer "F.Cu") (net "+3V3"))
 (segment (start 142 93.5) (end 143.275 94.775) (width 0.2) (layer "F.Cu") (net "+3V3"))
 (segment (start 128.943316 105.946926) (end 140.396926 105.946926) (width 0.2) (layer "F.Cu") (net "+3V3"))
 (segment (start 143.275 94.775) (end 143.275 106.275) (width 0.2) (layer "F.Cu") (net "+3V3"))
 (segment (start 143.275 66.775) (end 143.275 78.175) (width 0.2) (layer "F.Cu") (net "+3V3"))
 (segment (start 104.21697 113.326926) (end 92 101.109956) (width 0.2) (layer "F.Cu") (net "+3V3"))
 (segment (start 92 115) (end 90.5 113.5) (width 0.2) (layer "F.Cu") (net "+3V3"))
 (segment (start 90.725 99.725) (end 90.725 88.021926) (width 0.2) (layer "F.Cu") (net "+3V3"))
 (segment (start 90.725 73.971926) (end 92 72.696926) (width 0.2) (layer "F.Cu") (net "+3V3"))
 (segment (start 143.275 106.275) (end 142 107.55) (width 0.2) (layer "F.Cu") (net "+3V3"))
 (segment (start 143.275 122.775) (end 143.275 134.225) (width 0.2) (layer "F.Cu") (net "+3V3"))
 (segment (start 142 79.45) (end 143.275 80.725) (width 0.2) (layer "F.Cu") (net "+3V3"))
 (segment (start 142 84.45) (end 140.5 85.95) (width 0.2) (layer "F.Cu") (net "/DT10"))
 (segment (start 140.5 85.95) (end 140.5 91.610242) (width 0.2) (layer "F.Cu") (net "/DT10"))
 (segment (start 140.5 91.610242) (end 130.093316 102.016926) (width 0.2) (layer "F.Cu") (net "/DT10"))
 (segment (start 140.725 83.765242) (end 130.093316 94.396926) (width 0.2) (layer "F.Cu") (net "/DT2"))
 (segment (start 142 70.5) (end 140.725 71.775) (width 0.2) (layer "F.Cu") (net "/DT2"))
 (segment (start 140.725 71.775) (end 140.725 83.765242) (width 0.2) (layer "F.Cu") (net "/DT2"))
 (segment (start 142 126.5) (end 139 123.5) (width 0.2) (layer "F.Cu") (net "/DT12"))
 (segment (start 139 123.5) (end 139 118.54361) (width 0.2) (layer "F.Cu") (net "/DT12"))
 (segment (start 139 118.54361) (end 130.093316 109.636926) (width 0.2) (layer "F.Cu") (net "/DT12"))
 (segment (start 103.030242 124) (end 104.693316 122.336926) (width 0.2) (layer "F.Cu") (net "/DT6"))
 (segment (start 92 124) (end 103.030242 124) (width 0.2) (layer "F.Cu") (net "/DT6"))
 (segment (start 142 98.5) (end 136.150242 98.5) (width 0.2) (layer "F.Cu") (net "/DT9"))
 (segment (start 136.150242 98.5) (end 130.093316 104.556926) (width 0.2) (layer "F.Cu") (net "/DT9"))
 (segment (start 142 112.55) (end 135.54639 112.55) (width 0.2) (layer "F.Cu") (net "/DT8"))
 (segment (start 135.54639 112.55) (end 130.093316 107.096926) (width 0.2) (layer "F.Cu") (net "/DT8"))
 (segment (start 131.243316 129.743316) (end 131.243316 113.326926) (width 0.2) (layer "F.Cu") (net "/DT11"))
 (segment (start 142 140.5) (end 131.243316 129.743316) (width 0.2) (layer "F.Cu") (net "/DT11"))
 (segment (start 131.243316 113.326926) (end 130.093316 112.176926) (width 0.2) (layer "F.Cu") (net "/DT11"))
 (segment (start 100.5 90.246926) (end 100.5 105.44361) (width 0.2) (layer "F.Cu") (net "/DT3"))
 (segment (start 92 81.746926) (end 100.5 90.246926) (width 0.2) (layer "F.Cu") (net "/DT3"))
 (segment (start 100.5 105.44361) (end 104.693316 109.636926) (width 0.2) (layer "F.Cu") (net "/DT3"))
 (segment (start 92 67.696926) (end 101 76.696926) (width 0.2) (layer "F.Cu") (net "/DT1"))
 (segment (start 101 76.696926) (end 101 95.78361) (width 0.2) (layer "F.Cu") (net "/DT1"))
 (segment (start 101 95.78361) (end 104.693316 99.476926) (width 0.2) (layer "F.Cu") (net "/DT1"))
 (segment (start 99.97639 110) (end 104.693316 114.716926) (width 0.2) (layer "F.Cu") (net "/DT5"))
 (segment (start 92 110) (end 99.97639 110) (width 0.2) (layer "F.Cu") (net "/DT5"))
 (segment (start 100.1 104.1) (end 100.1 107.58361) (width 0.2) (layer "F.Cu") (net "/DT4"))
 (segment (start 100.1 107.58361) (end 104.693316 112.176926) (width 0.2) (layer "F.Cu") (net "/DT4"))
 (segment (start 92 96) (end 100.1 104.1) (width 0.2) (layer "F.Cu") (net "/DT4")))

